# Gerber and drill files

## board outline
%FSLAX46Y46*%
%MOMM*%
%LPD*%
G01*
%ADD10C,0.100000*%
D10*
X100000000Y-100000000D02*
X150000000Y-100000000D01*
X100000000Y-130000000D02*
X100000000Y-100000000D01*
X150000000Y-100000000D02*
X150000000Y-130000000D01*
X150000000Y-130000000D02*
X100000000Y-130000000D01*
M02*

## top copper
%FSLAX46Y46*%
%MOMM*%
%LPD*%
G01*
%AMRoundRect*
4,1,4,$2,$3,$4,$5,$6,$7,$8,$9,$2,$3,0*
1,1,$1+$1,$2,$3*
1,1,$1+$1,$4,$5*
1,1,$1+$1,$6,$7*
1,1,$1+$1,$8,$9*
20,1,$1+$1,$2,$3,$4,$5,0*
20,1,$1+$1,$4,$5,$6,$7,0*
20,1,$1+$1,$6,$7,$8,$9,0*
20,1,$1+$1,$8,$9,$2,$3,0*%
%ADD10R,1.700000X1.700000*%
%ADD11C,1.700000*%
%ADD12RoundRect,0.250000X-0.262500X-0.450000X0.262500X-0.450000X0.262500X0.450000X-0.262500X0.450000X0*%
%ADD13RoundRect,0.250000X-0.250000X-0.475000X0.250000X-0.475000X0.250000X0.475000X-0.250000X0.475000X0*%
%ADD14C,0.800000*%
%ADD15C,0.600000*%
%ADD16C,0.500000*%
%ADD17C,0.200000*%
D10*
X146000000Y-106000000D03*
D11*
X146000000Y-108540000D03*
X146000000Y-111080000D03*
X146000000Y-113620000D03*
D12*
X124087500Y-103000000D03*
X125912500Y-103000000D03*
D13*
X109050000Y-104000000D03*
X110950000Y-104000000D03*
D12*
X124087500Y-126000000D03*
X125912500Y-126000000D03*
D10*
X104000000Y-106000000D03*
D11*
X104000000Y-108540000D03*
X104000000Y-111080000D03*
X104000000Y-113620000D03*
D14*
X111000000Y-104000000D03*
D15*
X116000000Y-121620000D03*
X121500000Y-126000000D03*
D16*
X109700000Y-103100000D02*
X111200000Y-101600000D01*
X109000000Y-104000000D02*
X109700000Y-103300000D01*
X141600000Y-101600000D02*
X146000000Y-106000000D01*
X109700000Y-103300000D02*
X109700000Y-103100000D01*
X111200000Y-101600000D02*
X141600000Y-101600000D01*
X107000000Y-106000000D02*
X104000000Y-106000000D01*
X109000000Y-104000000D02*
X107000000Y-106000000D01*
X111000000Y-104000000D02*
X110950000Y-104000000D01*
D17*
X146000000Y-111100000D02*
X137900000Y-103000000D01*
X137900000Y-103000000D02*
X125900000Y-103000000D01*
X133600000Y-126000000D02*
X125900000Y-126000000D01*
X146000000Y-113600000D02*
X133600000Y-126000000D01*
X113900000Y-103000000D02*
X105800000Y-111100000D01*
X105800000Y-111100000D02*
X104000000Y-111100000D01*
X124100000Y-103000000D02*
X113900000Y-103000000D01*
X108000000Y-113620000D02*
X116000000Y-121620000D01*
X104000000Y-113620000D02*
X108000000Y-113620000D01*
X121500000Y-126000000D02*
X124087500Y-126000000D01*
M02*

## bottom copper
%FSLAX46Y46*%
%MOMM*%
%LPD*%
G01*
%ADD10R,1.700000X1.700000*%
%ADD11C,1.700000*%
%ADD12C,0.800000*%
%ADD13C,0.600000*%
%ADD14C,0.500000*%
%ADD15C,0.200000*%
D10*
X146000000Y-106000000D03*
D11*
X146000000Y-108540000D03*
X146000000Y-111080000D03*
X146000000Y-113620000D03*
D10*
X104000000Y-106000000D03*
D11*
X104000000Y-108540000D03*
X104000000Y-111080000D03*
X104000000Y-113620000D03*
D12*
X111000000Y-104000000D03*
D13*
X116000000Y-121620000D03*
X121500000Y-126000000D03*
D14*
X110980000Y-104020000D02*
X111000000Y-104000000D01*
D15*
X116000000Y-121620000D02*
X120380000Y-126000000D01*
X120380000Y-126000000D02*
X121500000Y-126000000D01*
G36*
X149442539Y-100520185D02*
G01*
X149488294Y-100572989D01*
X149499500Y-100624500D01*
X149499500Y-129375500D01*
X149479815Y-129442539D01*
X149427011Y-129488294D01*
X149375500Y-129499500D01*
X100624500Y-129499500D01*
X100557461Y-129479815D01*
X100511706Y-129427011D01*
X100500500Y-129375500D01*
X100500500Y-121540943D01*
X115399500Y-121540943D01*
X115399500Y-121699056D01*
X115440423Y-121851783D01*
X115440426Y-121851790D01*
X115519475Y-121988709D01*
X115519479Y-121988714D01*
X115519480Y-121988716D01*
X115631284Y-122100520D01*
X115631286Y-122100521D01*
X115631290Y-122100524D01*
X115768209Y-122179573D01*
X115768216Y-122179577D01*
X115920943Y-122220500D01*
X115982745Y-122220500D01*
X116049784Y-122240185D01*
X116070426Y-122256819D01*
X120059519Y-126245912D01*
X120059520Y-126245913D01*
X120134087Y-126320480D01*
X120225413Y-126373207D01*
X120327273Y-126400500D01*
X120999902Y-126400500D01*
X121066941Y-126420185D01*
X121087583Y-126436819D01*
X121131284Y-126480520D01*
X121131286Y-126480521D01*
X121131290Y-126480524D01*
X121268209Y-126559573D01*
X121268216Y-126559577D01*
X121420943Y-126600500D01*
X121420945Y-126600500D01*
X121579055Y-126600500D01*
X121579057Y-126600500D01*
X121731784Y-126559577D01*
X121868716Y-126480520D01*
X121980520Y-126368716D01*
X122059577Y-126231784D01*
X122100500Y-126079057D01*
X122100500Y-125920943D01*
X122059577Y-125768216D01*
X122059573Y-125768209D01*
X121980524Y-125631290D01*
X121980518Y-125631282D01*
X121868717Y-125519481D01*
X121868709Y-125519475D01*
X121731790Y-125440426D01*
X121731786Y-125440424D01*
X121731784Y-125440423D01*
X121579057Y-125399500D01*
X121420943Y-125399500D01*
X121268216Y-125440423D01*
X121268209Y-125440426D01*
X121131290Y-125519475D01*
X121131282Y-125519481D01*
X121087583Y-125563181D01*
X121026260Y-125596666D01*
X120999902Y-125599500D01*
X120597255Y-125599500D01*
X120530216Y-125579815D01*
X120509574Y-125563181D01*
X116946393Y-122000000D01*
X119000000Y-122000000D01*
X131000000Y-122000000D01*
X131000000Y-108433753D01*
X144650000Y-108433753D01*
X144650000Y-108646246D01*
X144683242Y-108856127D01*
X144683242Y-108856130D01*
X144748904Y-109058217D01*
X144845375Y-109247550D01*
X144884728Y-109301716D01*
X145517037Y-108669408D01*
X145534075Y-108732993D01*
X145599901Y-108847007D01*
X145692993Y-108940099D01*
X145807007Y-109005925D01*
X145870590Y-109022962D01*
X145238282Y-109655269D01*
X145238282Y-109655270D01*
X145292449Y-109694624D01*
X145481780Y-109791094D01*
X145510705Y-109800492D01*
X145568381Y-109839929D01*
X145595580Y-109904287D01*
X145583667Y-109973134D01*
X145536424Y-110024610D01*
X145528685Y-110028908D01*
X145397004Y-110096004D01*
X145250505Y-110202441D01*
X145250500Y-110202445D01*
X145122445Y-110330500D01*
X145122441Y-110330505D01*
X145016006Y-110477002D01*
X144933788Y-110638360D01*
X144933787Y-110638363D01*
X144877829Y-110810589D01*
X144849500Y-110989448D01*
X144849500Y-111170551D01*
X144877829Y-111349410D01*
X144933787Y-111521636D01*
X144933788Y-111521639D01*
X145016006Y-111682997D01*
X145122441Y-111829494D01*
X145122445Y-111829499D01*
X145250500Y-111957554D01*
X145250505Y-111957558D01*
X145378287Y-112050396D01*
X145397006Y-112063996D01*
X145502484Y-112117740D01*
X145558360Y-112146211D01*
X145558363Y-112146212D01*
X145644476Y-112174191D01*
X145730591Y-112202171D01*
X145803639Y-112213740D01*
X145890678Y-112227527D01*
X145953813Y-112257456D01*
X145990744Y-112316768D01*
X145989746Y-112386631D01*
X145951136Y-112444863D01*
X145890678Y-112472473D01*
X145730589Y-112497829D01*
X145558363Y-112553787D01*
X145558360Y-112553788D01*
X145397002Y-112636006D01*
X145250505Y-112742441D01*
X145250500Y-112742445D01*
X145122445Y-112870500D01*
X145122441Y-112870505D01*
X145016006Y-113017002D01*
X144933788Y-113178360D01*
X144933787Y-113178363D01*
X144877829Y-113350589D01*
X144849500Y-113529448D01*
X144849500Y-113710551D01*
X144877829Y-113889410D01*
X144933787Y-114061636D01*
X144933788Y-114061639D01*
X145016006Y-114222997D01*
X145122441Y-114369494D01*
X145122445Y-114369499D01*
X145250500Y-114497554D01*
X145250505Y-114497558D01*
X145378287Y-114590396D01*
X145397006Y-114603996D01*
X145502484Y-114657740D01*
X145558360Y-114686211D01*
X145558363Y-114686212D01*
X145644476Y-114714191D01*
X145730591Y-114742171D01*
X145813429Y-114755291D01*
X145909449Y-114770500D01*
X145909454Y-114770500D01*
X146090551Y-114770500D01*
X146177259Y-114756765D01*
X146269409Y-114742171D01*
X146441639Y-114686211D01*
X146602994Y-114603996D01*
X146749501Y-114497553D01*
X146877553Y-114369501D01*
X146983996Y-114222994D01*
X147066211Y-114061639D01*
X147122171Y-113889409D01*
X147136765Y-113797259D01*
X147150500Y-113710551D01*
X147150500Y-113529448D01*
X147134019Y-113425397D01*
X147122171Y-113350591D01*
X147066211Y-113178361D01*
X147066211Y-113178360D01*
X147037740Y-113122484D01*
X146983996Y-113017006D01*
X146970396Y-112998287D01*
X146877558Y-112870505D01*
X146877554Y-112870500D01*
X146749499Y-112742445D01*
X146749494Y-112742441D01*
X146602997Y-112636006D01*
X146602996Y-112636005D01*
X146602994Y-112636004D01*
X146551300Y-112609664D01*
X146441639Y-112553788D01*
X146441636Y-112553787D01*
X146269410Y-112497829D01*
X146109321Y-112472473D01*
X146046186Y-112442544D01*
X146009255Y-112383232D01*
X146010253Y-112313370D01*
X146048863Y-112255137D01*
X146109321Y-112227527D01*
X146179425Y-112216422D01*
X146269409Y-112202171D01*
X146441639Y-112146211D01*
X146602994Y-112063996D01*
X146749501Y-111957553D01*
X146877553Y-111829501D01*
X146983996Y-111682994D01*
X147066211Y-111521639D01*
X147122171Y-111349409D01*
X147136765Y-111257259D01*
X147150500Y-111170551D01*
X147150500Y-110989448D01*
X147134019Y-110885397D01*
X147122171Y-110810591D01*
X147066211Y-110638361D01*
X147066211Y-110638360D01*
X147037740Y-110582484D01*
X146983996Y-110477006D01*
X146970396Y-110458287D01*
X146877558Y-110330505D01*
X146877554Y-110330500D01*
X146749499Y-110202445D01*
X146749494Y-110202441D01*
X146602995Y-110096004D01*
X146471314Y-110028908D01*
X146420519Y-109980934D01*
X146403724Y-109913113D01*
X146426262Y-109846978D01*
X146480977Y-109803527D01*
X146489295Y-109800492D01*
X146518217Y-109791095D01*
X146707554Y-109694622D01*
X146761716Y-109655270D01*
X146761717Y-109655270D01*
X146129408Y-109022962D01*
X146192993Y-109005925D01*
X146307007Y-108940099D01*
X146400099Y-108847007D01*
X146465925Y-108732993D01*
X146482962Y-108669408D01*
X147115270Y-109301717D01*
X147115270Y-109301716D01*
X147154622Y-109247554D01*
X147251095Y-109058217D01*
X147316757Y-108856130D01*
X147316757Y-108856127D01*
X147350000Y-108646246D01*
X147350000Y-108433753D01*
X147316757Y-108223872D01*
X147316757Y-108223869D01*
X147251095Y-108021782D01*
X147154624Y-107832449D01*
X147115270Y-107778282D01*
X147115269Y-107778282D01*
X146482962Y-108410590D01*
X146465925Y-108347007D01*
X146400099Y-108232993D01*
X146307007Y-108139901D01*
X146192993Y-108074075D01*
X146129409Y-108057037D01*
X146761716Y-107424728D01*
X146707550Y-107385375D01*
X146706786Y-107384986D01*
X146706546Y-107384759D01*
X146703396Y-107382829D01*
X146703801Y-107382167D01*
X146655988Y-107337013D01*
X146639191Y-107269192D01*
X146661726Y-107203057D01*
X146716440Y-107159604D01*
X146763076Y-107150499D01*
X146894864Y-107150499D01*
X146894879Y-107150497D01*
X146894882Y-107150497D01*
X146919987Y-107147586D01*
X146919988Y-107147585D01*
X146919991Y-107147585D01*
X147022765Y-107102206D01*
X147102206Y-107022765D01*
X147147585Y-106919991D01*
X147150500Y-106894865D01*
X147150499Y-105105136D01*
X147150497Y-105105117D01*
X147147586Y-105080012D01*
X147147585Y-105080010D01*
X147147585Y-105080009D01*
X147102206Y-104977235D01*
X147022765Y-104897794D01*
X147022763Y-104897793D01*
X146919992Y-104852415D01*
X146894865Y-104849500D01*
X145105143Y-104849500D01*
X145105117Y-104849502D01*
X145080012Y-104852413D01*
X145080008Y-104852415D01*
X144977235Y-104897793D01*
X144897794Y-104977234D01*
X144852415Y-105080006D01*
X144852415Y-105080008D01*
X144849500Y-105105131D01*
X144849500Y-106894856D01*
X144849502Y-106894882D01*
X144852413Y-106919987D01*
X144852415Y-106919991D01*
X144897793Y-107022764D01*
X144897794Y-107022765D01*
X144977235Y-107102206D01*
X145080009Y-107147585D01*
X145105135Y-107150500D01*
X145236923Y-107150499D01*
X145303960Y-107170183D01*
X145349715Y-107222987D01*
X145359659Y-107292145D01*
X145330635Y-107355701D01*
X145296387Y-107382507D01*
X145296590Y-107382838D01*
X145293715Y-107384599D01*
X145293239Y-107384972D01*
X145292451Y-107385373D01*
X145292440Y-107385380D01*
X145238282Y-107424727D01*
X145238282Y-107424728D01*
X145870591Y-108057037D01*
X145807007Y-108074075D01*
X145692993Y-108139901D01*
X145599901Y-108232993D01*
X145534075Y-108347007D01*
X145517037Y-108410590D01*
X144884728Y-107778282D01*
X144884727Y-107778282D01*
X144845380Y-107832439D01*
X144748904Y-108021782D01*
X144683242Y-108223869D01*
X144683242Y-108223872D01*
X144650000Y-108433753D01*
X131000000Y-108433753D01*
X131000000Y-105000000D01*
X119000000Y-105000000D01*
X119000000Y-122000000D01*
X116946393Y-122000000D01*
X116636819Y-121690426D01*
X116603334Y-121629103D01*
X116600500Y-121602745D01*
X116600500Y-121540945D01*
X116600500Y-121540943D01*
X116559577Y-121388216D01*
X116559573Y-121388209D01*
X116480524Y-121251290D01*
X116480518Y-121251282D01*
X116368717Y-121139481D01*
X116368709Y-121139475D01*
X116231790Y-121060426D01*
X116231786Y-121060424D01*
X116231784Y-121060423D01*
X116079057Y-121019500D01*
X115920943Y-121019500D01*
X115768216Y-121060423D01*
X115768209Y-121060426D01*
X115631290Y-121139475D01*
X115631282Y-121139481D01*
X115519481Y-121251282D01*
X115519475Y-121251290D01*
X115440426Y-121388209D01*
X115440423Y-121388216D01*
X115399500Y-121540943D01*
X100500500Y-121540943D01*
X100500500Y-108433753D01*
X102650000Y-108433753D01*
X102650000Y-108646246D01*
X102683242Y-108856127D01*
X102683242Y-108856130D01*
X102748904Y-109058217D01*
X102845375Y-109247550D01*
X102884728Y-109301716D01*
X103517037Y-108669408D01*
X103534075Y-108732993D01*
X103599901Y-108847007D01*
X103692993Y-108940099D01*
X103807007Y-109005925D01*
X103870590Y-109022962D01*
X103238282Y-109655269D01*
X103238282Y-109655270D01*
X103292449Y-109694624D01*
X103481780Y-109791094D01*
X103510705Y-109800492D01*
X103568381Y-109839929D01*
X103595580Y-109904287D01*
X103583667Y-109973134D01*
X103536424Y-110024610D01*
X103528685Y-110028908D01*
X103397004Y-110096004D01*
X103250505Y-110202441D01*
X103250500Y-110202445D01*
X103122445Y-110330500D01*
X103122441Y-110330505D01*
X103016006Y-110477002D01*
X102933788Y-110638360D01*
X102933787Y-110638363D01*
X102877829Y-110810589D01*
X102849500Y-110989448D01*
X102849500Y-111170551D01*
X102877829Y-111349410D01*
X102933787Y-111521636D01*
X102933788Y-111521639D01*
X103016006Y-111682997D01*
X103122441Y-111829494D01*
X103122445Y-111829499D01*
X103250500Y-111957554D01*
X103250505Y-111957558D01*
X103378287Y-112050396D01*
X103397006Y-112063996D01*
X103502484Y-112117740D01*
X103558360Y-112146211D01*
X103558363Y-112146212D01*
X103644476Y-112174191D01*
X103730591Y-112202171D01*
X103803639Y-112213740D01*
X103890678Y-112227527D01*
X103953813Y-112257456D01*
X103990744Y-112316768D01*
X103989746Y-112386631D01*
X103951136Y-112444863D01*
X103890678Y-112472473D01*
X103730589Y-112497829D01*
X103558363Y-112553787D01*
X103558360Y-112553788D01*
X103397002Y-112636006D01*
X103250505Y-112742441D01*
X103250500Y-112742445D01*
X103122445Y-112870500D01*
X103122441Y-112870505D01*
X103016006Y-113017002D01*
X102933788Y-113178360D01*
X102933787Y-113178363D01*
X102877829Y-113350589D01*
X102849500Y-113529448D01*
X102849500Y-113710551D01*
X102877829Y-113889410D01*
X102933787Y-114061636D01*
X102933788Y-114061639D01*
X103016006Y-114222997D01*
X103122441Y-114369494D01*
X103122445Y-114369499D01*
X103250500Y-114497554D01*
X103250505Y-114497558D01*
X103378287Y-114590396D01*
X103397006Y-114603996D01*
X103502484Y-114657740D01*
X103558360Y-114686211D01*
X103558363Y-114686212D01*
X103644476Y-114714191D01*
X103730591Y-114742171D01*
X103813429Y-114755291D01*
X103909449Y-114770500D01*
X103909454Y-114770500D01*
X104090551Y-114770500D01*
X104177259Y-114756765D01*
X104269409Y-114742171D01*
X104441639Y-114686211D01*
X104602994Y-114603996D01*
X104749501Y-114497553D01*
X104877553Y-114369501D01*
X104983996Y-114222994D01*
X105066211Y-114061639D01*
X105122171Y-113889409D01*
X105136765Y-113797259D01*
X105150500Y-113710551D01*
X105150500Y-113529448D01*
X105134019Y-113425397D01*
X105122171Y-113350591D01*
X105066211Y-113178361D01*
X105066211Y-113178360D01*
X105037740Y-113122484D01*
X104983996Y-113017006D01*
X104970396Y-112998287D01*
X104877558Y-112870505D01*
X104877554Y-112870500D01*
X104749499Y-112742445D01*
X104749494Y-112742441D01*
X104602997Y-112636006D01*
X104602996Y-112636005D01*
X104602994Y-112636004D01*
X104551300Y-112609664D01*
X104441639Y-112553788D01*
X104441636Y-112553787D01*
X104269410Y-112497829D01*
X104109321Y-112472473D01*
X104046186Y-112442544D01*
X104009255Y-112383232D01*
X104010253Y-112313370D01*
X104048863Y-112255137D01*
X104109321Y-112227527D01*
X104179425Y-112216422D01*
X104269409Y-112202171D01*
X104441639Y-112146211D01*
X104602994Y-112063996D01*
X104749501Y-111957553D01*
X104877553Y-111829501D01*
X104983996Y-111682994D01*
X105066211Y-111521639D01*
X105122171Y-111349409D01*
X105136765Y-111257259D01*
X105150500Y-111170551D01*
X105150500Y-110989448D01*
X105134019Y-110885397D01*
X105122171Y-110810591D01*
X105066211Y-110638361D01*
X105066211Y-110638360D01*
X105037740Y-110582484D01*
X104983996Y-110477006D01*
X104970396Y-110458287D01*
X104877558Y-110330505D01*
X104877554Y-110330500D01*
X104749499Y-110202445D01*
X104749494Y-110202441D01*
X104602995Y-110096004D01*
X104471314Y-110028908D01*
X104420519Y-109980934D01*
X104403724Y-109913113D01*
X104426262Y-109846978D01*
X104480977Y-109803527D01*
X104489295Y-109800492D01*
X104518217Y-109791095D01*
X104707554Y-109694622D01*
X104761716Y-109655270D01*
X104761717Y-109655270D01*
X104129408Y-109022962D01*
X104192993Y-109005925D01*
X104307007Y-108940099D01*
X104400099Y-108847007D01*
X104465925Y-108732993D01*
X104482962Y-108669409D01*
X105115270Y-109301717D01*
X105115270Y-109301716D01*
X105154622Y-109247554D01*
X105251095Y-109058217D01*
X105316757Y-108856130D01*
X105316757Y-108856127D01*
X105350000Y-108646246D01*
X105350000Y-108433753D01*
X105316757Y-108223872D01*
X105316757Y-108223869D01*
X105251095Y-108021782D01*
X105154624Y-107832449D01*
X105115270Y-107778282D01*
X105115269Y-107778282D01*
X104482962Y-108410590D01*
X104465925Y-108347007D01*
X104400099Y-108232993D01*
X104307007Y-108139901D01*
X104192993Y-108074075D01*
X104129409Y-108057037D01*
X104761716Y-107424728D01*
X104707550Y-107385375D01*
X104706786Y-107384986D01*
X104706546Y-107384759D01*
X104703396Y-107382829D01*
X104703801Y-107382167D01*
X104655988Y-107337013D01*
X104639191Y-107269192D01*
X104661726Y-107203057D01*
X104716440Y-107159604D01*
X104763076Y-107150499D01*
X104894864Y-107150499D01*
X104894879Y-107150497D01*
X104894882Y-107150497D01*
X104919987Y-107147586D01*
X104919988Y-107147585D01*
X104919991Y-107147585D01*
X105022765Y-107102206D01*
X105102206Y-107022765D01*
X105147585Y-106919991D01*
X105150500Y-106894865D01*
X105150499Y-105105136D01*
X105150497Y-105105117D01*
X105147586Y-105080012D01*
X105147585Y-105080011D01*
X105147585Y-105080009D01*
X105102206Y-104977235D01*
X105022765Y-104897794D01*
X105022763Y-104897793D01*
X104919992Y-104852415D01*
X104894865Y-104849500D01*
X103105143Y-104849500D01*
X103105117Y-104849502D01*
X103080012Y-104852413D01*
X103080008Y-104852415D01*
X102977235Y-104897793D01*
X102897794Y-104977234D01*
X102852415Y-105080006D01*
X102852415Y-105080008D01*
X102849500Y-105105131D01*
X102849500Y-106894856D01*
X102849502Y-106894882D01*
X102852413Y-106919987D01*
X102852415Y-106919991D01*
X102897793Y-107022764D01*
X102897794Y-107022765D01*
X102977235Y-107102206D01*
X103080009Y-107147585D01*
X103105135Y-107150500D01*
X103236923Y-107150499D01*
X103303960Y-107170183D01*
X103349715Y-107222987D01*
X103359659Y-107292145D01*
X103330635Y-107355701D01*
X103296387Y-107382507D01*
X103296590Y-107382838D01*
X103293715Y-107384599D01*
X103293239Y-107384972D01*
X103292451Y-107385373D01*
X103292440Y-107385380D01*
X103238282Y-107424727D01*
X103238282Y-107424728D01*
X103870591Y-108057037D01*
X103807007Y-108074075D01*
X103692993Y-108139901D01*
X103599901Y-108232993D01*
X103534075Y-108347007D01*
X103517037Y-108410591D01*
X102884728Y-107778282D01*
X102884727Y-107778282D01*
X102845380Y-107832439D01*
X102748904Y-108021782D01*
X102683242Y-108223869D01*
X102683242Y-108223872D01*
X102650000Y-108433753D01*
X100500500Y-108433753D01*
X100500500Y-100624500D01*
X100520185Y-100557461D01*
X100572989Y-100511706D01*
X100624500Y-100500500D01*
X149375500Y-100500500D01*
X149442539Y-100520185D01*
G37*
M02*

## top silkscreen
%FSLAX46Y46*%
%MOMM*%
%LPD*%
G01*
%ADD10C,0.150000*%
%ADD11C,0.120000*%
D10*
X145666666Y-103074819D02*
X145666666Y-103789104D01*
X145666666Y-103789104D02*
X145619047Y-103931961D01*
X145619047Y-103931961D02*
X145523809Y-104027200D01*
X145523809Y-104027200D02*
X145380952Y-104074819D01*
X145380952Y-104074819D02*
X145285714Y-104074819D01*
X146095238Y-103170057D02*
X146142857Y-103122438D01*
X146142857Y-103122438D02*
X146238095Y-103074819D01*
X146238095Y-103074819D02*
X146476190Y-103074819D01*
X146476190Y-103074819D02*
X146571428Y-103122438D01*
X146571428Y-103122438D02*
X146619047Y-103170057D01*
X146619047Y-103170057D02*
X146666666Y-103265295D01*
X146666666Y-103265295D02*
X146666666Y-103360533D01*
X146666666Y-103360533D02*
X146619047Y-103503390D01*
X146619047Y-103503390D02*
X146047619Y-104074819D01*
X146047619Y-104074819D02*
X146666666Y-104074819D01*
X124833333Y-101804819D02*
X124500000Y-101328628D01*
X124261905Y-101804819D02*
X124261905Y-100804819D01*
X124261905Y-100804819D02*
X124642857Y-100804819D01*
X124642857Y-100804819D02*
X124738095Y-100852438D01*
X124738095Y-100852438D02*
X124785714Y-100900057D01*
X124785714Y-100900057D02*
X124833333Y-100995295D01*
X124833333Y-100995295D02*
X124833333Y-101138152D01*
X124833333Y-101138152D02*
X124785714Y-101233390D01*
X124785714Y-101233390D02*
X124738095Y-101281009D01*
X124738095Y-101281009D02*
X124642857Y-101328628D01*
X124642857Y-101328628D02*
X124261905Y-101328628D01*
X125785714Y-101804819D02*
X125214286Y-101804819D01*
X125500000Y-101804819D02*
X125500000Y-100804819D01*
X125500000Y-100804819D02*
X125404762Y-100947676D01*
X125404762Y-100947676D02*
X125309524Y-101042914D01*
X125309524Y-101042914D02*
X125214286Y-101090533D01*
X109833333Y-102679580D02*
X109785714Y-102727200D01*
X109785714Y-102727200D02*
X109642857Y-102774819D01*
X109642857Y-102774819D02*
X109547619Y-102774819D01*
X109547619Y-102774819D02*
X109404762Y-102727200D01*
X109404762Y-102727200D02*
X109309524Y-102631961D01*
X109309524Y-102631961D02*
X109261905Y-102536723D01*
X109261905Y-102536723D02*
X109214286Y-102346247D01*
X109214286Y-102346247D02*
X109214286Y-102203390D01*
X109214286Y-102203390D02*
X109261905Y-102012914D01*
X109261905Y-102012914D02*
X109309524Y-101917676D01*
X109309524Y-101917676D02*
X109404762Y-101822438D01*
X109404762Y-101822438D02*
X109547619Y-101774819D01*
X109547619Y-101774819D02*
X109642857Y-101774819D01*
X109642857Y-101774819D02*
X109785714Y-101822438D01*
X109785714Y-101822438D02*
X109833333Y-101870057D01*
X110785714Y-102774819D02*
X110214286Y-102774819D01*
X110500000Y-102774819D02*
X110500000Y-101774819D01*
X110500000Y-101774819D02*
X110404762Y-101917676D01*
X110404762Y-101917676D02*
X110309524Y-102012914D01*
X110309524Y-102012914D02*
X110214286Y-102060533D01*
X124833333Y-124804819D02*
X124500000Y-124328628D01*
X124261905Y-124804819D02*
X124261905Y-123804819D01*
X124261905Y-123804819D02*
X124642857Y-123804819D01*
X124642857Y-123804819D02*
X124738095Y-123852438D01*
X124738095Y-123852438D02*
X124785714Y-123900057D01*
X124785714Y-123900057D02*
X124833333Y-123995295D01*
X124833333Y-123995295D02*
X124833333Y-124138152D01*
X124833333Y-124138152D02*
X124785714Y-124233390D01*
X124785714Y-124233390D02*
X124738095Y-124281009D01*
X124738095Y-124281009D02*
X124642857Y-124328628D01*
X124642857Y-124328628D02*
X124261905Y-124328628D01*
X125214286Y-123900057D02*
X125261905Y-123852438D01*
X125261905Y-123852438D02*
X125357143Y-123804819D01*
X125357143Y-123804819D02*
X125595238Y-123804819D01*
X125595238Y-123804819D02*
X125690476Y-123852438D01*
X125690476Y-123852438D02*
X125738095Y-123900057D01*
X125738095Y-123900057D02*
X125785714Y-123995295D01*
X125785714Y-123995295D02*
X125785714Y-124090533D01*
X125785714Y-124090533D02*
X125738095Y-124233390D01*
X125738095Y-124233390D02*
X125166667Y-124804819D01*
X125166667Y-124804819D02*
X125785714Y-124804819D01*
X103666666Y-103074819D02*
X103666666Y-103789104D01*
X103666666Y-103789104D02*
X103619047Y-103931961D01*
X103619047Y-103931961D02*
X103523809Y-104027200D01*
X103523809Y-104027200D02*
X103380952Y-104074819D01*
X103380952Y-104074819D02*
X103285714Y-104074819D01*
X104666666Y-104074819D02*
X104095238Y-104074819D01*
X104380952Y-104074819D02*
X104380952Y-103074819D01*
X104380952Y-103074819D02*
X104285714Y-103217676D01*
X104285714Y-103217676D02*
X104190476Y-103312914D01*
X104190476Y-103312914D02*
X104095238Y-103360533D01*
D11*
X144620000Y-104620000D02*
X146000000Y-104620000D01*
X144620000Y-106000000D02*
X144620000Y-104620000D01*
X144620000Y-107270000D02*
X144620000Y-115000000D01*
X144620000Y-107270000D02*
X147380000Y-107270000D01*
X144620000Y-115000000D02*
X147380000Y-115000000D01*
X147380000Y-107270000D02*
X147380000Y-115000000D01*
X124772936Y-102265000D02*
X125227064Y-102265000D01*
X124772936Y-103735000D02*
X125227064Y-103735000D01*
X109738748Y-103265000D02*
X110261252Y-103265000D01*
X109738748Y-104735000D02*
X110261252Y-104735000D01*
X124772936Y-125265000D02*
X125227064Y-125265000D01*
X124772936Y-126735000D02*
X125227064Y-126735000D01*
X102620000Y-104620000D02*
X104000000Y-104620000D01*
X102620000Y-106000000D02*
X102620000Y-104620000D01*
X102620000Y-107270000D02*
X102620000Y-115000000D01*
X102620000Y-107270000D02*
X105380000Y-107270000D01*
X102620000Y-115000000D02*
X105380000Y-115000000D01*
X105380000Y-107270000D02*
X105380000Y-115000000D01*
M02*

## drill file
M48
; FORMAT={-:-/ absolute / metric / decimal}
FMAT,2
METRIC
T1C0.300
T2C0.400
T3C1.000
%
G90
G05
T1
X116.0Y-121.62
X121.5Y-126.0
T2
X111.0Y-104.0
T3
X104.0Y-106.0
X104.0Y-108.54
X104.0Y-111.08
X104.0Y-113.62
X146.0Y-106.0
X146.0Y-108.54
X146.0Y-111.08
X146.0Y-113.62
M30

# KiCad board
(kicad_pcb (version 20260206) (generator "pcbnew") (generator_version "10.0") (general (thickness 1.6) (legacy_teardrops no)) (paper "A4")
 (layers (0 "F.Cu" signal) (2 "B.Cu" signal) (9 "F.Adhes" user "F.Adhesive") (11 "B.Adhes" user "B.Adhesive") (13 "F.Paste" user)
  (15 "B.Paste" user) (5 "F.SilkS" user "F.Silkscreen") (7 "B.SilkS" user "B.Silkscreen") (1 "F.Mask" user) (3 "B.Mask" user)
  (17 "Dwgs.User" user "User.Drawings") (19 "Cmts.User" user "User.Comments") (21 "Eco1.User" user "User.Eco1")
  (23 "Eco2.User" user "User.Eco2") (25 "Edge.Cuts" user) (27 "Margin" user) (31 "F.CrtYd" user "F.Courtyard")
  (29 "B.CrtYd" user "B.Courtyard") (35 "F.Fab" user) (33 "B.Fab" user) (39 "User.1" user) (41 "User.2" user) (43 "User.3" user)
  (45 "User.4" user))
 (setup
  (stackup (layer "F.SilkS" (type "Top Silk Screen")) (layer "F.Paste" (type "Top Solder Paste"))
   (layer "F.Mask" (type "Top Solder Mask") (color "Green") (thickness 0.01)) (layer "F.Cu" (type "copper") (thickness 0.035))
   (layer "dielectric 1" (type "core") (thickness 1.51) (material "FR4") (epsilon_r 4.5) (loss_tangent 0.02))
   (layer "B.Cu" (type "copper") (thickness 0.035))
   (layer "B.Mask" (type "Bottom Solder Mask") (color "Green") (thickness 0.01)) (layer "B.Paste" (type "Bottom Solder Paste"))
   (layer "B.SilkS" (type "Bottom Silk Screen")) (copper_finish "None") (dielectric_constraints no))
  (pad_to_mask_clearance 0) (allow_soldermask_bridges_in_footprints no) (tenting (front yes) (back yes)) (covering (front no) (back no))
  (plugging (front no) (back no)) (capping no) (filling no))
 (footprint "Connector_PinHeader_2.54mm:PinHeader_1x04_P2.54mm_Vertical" (layer "F.Cu") (at 146 106)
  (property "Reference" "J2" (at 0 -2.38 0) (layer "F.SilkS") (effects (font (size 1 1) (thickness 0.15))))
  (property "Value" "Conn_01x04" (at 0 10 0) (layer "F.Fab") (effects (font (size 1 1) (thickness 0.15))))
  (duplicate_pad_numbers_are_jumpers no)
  (fp_line (start -1.38 -1.38) (end 0 -1.38) (stroke (width 0.12) (type solid)) (layer "F.SilkS"))
  (fp_line (start -1.38 0) (end -1.38 -1.38) (stroke (width 0.12) (type solid)) (layer "F.SilkS"))
  (fp_line (start -1.38 1.27) (end -1.38 9) (stroke (width 0.12) (type solid)) (layer "F.SilkS"))
  (fp_line (start -1.38 1.27) (end 1.38 1.27) (stroke (width 0.12) (type solid)) (layer "F.SilkS"))
  (fp_line (start -1.38 9) (end 1.38 9) (stroke (width 0.12) (type solid)) (layer "F.SilkS"))
  (fp_line (start 1.38 1.27) (end 1.38 9) (stroke (width 0.12) (type solid)) (layer "F.SilkS"))
  (pad "1" thru_hole rect (at 0 0) (size 1.7 1.7) (drill 1) (layers "*.Cu" "*.Mask") (remove_unused_layers no) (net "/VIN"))
  (pad "2" thru_hole circle (at 0 2.54) (size 1.7 1.7) (drill 1) (layers "*.Cu" "*.Mask") (remove_unused_layers no) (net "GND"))
  (pad "3" thru_hole circle (at 0 5.08) (size 1.7 1.7) (drill 1) (layers "*.Cu" "*.Mask") (remove_unused_layers no) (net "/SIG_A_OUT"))
  (pad "4" thru_hole circle (at 0 7.62) (size 1.7 1.7) (drill 1) (layers "*.Cu" "*.Mask") (remove_unused_layers no) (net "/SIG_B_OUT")))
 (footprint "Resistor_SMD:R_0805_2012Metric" (layer "F.Cu") (at 125 103)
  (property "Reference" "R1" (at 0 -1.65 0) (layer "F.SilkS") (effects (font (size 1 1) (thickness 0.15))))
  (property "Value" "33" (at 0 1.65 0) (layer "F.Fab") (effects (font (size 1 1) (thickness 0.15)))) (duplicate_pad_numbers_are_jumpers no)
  (fp_line (start -0.227064 -0.735) (end 0.227064 -0.735) (stroke (width 0.12) (type solid)) (layer "F.SilkS"))
  (fp_line (start -0.227064 0.735) (end 0.227064 0.735) (stroke (width 0.12) (type solid)) (layer "F.SilkS"))
  (pad "1" smd roundrect (at -0.9125 0) (size 1.025 1.4) (layers "F.Cu" "F.Mask" "F.Paste") (roundrect_rratio 0.243902) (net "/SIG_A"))
  (pad "2" smd roundrect (at 0.9125 0) (size 1.025 1.4) (layers "F.Cu" "F.Mask" "F.Paste") (roundrect_rratio 0.243902) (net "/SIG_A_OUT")))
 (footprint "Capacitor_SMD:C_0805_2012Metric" (layer "F.Cu") (at 110 104)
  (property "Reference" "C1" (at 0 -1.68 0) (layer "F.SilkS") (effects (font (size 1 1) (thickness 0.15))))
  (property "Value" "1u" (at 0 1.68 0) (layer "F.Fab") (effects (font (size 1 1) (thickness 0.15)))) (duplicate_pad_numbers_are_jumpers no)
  (fp_line (start -0.261252 -0.735) (end 0.261252 -0.735) (stroke (width 0.12) (type solid)) (layer "F.SilkS"))
  (fp_line (start -0.261252 0.735) (end 0.261252 0.735) (stroke (width 0.12) (type solid)) (layer "F.SilkS"))
  (pad "1" smd roundrect (at -0.95 0) (size 1 1.45) (layers "F.Cu" "F.Mask" "F.Paste") (roundrect_rratio 0.25) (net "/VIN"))
  (pad "2" smd roundrect (at 0.95 0) (size 1 1.45) (layers "F.Cu" "F.Mask" "F.Paste") (roundrect_rratio 0.25) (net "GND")))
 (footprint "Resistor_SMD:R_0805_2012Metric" (layer "F.Cu") (at 125 126)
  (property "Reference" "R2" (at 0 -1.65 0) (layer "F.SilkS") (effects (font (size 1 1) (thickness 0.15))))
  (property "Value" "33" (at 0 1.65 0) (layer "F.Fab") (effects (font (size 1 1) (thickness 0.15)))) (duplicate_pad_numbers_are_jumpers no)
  (fp_line (start -0.227064 -0.735) (end 0.227064 -0.735) (stroke (width 0.12) (type solid)) (layer "F.SilkS"))
  (fp_line (start -0.227064 0.735) (end 0.227064 0.735) (stroke (width 0.12) (type solid)) (layer "F.SilkS"))
  (pad "1" smd roundrect (at -0.9125 0) (size 1.025 1.4) (layers "F.Cu" "F.Mask" "F.Paste") (roundrect_rratio 0.243902) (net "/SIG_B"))
  (pad "2" smd roundrect (at 0.9125 0) (size 1.025 1.4) (layers "F.Cu" "F.Mask" "F.Paste") (roundrect_rratio 0.243902) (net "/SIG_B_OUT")))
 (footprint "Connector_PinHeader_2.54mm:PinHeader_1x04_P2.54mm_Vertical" (layer "F.Cu") (at 104 106)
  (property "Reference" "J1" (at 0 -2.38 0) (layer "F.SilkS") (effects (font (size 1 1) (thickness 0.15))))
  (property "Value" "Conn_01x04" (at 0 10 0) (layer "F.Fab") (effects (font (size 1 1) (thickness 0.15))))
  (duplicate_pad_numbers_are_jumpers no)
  (fp_line (start -1.38 -1.38) (end 0 -1.38) (stroke (width 0.12) (type solid)) (layer "F.SilkS"))
  (fp_line (start -1.38 0) (end -1.38 -1.38) (stroke (width 0.12) (type solid)) (layer "F.SilkS"))
  (fp_line (start -1.38 1.27) (end -1.38 9) (stroke (width 0.12) (type solid)) (layer "F.SilkS"))
  (fp_line (start -1.38 1.27) (end 1.38 1.27) (stroke (width 0.12) (type solid)) (layer "F.SilkS"))
  (fp_line (start -1.38 9) (end 1.38 9) (stroke (width 0.12) (type solid)) (layer "F.SilkS"))
  (fp_line (start 1.38 1.27) (end 1.38 9) (stroke (width 0.12) (type solid)) (layer "F.SilkS"))
  (pad "1" thru_hole rect (at 0 0) (size 1.7 1.7) (drill 1) (layers "*.Cu" "*.Mask") (remove_unused_layers no) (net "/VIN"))
  (pad "2" thru_hole circle (at 0 2.54) (size 1.7 1.7) (drill 1) (layers "*.Cu" "*.Mask") (remove_unused_layers no) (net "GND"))
  (pad "3" thru_hole circle (at 0 5.08) (size 1.7 1.7) (drill 1) (layers "*.Cu" "*.Mask") (remove_unused_layers no) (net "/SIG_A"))
  (pad "4" thru_hole circle (at 0 7.62) (size 1.7 1.7) (drill 1) (layers "*.Cu" "*.Mask") (remove_unused_layers no) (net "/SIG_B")))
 (gr_line (start 100 100) (end 150 100) (stroke (width 0.1) (type default)) (layer "Edge.Cuts"))
 (gr_line (start 100 130) (end 100 100) (stroke (width 0.1) (type default)) (layer "Edge.Cuts"))
 (gr_line (start 150 100) (end 150 130) (stroke (width 0.1) (type default)) (layer "Edge.Cuts"))
 (gr_line (start 150 130) (end 100 130) (stroke (width 0.1) (type default)) (layer "Edge.Cuts"))
 (segment (start 109.7 103.1) (end 111.2 101.6) (width 0.5) (layer "F.Cu") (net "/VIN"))
 (segment (start 109 104) (end 109.7 103.3) (width 0.5) (layer "F.Cu") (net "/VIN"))
 (segment (start 141.6 101.6) (end 146 106) (width 0.5) (layer "F.Cu") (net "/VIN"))
 (segment (start 109.7 103.3) (end 109.7 103.1) (width 0.5) (layer "F.Cu") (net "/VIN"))
 (segment (start 111.2 101.6) (end 141.6 101.6) (width 0.5) (layer "F.Cu") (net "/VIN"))
 (segment (start 107 106) (end 104 106) (width 0.5) (layer "F.Cu") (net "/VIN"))
 (segment (start 109 104) (end 107 106) (width 0.5) (layer "F.Cu") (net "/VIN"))
 (segment (start 111 104) (end 110.95 104) (width 0.5) (layer "F.Cu") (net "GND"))
 (via (at 111 104) (size 0.8) (drill 0.4) (layers "F.Cu" "B.Cu") (capping yes) (filling yes) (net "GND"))
 (segment (start 110.98 104.02) (end 111 104) (width 0.5) (layer "B.Cu") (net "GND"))
 (segment (start 146 111.1) (end 137.9 103) (width 0.2) (layer "F.Cu") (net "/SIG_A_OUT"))
 (segment (start 137.9 103) (end 125.9 103) (width 0.2) (layer "F.Cu") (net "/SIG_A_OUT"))
 (segment (start 133.6 126) (end 125.9 126) (width 0.2) (layer "F.Cu") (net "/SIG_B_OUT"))
 (segment (start 146 113.6) (end 133.6 126) (width 0.2) (layer "F.Cu") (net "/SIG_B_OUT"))
 (segment (start 113.9 103) (end 105.8 111.1) (width 0.2) (layer "F.Cu") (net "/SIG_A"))
 (segment (start 105.8 111.1) (end 104 111.1) (width 0.2) (layer "F.Cu") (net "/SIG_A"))
 (segment (start 124.1 103) (end 113.9 103) (width 0.2) (layer "F.Cu") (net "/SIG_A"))
 (segment (start 108 113.62) (end 116 121.62) (width 0.2) (locked yes) (layer "F.Cu") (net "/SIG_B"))
 (segment (start 104 113.62) (end 108 113.62) (width 0.2) (locked yes) (layer "F.Cu") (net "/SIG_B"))
 (segment (start 121.5 126) (end 124.0875 126) (width 0.2) (locked yes) (layer "F.Cu") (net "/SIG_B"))
 (via (at 116 121.62) (size 0.6) (drill 0.3) (layers "F.Cu" "B.Cu") (locked yes) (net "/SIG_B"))
 (via (at 121.5 126) (size 0.6) (drill 0.3) (layers "F.Cu" "B.Cu") (locked yes) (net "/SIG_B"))
 (segment (start 116 121.62) (end 120.38 126) (width 0.2) (locked yes) (layer "B.Cu") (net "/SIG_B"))
 (segment (start 120.38 126) (end 121.5 126) (width 0.2) (locked yes) (layer "B.Cu") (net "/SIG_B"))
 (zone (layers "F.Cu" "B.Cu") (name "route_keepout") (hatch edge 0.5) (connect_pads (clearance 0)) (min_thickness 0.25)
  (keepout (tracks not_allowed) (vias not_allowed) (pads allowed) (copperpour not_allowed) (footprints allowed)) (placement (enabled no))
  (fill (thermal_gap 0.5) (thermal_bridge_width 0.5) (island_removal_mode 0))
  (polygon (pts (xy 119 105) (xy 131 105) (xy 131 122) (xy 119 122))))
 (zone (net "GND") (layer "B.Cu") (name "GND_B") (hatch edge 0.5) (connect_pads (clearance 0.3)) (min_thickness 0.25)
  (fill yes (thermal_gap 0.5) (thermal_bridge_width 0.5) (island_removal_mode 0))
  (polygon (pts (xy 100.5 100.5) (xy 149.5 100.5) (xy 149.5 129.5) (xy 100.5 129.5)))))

